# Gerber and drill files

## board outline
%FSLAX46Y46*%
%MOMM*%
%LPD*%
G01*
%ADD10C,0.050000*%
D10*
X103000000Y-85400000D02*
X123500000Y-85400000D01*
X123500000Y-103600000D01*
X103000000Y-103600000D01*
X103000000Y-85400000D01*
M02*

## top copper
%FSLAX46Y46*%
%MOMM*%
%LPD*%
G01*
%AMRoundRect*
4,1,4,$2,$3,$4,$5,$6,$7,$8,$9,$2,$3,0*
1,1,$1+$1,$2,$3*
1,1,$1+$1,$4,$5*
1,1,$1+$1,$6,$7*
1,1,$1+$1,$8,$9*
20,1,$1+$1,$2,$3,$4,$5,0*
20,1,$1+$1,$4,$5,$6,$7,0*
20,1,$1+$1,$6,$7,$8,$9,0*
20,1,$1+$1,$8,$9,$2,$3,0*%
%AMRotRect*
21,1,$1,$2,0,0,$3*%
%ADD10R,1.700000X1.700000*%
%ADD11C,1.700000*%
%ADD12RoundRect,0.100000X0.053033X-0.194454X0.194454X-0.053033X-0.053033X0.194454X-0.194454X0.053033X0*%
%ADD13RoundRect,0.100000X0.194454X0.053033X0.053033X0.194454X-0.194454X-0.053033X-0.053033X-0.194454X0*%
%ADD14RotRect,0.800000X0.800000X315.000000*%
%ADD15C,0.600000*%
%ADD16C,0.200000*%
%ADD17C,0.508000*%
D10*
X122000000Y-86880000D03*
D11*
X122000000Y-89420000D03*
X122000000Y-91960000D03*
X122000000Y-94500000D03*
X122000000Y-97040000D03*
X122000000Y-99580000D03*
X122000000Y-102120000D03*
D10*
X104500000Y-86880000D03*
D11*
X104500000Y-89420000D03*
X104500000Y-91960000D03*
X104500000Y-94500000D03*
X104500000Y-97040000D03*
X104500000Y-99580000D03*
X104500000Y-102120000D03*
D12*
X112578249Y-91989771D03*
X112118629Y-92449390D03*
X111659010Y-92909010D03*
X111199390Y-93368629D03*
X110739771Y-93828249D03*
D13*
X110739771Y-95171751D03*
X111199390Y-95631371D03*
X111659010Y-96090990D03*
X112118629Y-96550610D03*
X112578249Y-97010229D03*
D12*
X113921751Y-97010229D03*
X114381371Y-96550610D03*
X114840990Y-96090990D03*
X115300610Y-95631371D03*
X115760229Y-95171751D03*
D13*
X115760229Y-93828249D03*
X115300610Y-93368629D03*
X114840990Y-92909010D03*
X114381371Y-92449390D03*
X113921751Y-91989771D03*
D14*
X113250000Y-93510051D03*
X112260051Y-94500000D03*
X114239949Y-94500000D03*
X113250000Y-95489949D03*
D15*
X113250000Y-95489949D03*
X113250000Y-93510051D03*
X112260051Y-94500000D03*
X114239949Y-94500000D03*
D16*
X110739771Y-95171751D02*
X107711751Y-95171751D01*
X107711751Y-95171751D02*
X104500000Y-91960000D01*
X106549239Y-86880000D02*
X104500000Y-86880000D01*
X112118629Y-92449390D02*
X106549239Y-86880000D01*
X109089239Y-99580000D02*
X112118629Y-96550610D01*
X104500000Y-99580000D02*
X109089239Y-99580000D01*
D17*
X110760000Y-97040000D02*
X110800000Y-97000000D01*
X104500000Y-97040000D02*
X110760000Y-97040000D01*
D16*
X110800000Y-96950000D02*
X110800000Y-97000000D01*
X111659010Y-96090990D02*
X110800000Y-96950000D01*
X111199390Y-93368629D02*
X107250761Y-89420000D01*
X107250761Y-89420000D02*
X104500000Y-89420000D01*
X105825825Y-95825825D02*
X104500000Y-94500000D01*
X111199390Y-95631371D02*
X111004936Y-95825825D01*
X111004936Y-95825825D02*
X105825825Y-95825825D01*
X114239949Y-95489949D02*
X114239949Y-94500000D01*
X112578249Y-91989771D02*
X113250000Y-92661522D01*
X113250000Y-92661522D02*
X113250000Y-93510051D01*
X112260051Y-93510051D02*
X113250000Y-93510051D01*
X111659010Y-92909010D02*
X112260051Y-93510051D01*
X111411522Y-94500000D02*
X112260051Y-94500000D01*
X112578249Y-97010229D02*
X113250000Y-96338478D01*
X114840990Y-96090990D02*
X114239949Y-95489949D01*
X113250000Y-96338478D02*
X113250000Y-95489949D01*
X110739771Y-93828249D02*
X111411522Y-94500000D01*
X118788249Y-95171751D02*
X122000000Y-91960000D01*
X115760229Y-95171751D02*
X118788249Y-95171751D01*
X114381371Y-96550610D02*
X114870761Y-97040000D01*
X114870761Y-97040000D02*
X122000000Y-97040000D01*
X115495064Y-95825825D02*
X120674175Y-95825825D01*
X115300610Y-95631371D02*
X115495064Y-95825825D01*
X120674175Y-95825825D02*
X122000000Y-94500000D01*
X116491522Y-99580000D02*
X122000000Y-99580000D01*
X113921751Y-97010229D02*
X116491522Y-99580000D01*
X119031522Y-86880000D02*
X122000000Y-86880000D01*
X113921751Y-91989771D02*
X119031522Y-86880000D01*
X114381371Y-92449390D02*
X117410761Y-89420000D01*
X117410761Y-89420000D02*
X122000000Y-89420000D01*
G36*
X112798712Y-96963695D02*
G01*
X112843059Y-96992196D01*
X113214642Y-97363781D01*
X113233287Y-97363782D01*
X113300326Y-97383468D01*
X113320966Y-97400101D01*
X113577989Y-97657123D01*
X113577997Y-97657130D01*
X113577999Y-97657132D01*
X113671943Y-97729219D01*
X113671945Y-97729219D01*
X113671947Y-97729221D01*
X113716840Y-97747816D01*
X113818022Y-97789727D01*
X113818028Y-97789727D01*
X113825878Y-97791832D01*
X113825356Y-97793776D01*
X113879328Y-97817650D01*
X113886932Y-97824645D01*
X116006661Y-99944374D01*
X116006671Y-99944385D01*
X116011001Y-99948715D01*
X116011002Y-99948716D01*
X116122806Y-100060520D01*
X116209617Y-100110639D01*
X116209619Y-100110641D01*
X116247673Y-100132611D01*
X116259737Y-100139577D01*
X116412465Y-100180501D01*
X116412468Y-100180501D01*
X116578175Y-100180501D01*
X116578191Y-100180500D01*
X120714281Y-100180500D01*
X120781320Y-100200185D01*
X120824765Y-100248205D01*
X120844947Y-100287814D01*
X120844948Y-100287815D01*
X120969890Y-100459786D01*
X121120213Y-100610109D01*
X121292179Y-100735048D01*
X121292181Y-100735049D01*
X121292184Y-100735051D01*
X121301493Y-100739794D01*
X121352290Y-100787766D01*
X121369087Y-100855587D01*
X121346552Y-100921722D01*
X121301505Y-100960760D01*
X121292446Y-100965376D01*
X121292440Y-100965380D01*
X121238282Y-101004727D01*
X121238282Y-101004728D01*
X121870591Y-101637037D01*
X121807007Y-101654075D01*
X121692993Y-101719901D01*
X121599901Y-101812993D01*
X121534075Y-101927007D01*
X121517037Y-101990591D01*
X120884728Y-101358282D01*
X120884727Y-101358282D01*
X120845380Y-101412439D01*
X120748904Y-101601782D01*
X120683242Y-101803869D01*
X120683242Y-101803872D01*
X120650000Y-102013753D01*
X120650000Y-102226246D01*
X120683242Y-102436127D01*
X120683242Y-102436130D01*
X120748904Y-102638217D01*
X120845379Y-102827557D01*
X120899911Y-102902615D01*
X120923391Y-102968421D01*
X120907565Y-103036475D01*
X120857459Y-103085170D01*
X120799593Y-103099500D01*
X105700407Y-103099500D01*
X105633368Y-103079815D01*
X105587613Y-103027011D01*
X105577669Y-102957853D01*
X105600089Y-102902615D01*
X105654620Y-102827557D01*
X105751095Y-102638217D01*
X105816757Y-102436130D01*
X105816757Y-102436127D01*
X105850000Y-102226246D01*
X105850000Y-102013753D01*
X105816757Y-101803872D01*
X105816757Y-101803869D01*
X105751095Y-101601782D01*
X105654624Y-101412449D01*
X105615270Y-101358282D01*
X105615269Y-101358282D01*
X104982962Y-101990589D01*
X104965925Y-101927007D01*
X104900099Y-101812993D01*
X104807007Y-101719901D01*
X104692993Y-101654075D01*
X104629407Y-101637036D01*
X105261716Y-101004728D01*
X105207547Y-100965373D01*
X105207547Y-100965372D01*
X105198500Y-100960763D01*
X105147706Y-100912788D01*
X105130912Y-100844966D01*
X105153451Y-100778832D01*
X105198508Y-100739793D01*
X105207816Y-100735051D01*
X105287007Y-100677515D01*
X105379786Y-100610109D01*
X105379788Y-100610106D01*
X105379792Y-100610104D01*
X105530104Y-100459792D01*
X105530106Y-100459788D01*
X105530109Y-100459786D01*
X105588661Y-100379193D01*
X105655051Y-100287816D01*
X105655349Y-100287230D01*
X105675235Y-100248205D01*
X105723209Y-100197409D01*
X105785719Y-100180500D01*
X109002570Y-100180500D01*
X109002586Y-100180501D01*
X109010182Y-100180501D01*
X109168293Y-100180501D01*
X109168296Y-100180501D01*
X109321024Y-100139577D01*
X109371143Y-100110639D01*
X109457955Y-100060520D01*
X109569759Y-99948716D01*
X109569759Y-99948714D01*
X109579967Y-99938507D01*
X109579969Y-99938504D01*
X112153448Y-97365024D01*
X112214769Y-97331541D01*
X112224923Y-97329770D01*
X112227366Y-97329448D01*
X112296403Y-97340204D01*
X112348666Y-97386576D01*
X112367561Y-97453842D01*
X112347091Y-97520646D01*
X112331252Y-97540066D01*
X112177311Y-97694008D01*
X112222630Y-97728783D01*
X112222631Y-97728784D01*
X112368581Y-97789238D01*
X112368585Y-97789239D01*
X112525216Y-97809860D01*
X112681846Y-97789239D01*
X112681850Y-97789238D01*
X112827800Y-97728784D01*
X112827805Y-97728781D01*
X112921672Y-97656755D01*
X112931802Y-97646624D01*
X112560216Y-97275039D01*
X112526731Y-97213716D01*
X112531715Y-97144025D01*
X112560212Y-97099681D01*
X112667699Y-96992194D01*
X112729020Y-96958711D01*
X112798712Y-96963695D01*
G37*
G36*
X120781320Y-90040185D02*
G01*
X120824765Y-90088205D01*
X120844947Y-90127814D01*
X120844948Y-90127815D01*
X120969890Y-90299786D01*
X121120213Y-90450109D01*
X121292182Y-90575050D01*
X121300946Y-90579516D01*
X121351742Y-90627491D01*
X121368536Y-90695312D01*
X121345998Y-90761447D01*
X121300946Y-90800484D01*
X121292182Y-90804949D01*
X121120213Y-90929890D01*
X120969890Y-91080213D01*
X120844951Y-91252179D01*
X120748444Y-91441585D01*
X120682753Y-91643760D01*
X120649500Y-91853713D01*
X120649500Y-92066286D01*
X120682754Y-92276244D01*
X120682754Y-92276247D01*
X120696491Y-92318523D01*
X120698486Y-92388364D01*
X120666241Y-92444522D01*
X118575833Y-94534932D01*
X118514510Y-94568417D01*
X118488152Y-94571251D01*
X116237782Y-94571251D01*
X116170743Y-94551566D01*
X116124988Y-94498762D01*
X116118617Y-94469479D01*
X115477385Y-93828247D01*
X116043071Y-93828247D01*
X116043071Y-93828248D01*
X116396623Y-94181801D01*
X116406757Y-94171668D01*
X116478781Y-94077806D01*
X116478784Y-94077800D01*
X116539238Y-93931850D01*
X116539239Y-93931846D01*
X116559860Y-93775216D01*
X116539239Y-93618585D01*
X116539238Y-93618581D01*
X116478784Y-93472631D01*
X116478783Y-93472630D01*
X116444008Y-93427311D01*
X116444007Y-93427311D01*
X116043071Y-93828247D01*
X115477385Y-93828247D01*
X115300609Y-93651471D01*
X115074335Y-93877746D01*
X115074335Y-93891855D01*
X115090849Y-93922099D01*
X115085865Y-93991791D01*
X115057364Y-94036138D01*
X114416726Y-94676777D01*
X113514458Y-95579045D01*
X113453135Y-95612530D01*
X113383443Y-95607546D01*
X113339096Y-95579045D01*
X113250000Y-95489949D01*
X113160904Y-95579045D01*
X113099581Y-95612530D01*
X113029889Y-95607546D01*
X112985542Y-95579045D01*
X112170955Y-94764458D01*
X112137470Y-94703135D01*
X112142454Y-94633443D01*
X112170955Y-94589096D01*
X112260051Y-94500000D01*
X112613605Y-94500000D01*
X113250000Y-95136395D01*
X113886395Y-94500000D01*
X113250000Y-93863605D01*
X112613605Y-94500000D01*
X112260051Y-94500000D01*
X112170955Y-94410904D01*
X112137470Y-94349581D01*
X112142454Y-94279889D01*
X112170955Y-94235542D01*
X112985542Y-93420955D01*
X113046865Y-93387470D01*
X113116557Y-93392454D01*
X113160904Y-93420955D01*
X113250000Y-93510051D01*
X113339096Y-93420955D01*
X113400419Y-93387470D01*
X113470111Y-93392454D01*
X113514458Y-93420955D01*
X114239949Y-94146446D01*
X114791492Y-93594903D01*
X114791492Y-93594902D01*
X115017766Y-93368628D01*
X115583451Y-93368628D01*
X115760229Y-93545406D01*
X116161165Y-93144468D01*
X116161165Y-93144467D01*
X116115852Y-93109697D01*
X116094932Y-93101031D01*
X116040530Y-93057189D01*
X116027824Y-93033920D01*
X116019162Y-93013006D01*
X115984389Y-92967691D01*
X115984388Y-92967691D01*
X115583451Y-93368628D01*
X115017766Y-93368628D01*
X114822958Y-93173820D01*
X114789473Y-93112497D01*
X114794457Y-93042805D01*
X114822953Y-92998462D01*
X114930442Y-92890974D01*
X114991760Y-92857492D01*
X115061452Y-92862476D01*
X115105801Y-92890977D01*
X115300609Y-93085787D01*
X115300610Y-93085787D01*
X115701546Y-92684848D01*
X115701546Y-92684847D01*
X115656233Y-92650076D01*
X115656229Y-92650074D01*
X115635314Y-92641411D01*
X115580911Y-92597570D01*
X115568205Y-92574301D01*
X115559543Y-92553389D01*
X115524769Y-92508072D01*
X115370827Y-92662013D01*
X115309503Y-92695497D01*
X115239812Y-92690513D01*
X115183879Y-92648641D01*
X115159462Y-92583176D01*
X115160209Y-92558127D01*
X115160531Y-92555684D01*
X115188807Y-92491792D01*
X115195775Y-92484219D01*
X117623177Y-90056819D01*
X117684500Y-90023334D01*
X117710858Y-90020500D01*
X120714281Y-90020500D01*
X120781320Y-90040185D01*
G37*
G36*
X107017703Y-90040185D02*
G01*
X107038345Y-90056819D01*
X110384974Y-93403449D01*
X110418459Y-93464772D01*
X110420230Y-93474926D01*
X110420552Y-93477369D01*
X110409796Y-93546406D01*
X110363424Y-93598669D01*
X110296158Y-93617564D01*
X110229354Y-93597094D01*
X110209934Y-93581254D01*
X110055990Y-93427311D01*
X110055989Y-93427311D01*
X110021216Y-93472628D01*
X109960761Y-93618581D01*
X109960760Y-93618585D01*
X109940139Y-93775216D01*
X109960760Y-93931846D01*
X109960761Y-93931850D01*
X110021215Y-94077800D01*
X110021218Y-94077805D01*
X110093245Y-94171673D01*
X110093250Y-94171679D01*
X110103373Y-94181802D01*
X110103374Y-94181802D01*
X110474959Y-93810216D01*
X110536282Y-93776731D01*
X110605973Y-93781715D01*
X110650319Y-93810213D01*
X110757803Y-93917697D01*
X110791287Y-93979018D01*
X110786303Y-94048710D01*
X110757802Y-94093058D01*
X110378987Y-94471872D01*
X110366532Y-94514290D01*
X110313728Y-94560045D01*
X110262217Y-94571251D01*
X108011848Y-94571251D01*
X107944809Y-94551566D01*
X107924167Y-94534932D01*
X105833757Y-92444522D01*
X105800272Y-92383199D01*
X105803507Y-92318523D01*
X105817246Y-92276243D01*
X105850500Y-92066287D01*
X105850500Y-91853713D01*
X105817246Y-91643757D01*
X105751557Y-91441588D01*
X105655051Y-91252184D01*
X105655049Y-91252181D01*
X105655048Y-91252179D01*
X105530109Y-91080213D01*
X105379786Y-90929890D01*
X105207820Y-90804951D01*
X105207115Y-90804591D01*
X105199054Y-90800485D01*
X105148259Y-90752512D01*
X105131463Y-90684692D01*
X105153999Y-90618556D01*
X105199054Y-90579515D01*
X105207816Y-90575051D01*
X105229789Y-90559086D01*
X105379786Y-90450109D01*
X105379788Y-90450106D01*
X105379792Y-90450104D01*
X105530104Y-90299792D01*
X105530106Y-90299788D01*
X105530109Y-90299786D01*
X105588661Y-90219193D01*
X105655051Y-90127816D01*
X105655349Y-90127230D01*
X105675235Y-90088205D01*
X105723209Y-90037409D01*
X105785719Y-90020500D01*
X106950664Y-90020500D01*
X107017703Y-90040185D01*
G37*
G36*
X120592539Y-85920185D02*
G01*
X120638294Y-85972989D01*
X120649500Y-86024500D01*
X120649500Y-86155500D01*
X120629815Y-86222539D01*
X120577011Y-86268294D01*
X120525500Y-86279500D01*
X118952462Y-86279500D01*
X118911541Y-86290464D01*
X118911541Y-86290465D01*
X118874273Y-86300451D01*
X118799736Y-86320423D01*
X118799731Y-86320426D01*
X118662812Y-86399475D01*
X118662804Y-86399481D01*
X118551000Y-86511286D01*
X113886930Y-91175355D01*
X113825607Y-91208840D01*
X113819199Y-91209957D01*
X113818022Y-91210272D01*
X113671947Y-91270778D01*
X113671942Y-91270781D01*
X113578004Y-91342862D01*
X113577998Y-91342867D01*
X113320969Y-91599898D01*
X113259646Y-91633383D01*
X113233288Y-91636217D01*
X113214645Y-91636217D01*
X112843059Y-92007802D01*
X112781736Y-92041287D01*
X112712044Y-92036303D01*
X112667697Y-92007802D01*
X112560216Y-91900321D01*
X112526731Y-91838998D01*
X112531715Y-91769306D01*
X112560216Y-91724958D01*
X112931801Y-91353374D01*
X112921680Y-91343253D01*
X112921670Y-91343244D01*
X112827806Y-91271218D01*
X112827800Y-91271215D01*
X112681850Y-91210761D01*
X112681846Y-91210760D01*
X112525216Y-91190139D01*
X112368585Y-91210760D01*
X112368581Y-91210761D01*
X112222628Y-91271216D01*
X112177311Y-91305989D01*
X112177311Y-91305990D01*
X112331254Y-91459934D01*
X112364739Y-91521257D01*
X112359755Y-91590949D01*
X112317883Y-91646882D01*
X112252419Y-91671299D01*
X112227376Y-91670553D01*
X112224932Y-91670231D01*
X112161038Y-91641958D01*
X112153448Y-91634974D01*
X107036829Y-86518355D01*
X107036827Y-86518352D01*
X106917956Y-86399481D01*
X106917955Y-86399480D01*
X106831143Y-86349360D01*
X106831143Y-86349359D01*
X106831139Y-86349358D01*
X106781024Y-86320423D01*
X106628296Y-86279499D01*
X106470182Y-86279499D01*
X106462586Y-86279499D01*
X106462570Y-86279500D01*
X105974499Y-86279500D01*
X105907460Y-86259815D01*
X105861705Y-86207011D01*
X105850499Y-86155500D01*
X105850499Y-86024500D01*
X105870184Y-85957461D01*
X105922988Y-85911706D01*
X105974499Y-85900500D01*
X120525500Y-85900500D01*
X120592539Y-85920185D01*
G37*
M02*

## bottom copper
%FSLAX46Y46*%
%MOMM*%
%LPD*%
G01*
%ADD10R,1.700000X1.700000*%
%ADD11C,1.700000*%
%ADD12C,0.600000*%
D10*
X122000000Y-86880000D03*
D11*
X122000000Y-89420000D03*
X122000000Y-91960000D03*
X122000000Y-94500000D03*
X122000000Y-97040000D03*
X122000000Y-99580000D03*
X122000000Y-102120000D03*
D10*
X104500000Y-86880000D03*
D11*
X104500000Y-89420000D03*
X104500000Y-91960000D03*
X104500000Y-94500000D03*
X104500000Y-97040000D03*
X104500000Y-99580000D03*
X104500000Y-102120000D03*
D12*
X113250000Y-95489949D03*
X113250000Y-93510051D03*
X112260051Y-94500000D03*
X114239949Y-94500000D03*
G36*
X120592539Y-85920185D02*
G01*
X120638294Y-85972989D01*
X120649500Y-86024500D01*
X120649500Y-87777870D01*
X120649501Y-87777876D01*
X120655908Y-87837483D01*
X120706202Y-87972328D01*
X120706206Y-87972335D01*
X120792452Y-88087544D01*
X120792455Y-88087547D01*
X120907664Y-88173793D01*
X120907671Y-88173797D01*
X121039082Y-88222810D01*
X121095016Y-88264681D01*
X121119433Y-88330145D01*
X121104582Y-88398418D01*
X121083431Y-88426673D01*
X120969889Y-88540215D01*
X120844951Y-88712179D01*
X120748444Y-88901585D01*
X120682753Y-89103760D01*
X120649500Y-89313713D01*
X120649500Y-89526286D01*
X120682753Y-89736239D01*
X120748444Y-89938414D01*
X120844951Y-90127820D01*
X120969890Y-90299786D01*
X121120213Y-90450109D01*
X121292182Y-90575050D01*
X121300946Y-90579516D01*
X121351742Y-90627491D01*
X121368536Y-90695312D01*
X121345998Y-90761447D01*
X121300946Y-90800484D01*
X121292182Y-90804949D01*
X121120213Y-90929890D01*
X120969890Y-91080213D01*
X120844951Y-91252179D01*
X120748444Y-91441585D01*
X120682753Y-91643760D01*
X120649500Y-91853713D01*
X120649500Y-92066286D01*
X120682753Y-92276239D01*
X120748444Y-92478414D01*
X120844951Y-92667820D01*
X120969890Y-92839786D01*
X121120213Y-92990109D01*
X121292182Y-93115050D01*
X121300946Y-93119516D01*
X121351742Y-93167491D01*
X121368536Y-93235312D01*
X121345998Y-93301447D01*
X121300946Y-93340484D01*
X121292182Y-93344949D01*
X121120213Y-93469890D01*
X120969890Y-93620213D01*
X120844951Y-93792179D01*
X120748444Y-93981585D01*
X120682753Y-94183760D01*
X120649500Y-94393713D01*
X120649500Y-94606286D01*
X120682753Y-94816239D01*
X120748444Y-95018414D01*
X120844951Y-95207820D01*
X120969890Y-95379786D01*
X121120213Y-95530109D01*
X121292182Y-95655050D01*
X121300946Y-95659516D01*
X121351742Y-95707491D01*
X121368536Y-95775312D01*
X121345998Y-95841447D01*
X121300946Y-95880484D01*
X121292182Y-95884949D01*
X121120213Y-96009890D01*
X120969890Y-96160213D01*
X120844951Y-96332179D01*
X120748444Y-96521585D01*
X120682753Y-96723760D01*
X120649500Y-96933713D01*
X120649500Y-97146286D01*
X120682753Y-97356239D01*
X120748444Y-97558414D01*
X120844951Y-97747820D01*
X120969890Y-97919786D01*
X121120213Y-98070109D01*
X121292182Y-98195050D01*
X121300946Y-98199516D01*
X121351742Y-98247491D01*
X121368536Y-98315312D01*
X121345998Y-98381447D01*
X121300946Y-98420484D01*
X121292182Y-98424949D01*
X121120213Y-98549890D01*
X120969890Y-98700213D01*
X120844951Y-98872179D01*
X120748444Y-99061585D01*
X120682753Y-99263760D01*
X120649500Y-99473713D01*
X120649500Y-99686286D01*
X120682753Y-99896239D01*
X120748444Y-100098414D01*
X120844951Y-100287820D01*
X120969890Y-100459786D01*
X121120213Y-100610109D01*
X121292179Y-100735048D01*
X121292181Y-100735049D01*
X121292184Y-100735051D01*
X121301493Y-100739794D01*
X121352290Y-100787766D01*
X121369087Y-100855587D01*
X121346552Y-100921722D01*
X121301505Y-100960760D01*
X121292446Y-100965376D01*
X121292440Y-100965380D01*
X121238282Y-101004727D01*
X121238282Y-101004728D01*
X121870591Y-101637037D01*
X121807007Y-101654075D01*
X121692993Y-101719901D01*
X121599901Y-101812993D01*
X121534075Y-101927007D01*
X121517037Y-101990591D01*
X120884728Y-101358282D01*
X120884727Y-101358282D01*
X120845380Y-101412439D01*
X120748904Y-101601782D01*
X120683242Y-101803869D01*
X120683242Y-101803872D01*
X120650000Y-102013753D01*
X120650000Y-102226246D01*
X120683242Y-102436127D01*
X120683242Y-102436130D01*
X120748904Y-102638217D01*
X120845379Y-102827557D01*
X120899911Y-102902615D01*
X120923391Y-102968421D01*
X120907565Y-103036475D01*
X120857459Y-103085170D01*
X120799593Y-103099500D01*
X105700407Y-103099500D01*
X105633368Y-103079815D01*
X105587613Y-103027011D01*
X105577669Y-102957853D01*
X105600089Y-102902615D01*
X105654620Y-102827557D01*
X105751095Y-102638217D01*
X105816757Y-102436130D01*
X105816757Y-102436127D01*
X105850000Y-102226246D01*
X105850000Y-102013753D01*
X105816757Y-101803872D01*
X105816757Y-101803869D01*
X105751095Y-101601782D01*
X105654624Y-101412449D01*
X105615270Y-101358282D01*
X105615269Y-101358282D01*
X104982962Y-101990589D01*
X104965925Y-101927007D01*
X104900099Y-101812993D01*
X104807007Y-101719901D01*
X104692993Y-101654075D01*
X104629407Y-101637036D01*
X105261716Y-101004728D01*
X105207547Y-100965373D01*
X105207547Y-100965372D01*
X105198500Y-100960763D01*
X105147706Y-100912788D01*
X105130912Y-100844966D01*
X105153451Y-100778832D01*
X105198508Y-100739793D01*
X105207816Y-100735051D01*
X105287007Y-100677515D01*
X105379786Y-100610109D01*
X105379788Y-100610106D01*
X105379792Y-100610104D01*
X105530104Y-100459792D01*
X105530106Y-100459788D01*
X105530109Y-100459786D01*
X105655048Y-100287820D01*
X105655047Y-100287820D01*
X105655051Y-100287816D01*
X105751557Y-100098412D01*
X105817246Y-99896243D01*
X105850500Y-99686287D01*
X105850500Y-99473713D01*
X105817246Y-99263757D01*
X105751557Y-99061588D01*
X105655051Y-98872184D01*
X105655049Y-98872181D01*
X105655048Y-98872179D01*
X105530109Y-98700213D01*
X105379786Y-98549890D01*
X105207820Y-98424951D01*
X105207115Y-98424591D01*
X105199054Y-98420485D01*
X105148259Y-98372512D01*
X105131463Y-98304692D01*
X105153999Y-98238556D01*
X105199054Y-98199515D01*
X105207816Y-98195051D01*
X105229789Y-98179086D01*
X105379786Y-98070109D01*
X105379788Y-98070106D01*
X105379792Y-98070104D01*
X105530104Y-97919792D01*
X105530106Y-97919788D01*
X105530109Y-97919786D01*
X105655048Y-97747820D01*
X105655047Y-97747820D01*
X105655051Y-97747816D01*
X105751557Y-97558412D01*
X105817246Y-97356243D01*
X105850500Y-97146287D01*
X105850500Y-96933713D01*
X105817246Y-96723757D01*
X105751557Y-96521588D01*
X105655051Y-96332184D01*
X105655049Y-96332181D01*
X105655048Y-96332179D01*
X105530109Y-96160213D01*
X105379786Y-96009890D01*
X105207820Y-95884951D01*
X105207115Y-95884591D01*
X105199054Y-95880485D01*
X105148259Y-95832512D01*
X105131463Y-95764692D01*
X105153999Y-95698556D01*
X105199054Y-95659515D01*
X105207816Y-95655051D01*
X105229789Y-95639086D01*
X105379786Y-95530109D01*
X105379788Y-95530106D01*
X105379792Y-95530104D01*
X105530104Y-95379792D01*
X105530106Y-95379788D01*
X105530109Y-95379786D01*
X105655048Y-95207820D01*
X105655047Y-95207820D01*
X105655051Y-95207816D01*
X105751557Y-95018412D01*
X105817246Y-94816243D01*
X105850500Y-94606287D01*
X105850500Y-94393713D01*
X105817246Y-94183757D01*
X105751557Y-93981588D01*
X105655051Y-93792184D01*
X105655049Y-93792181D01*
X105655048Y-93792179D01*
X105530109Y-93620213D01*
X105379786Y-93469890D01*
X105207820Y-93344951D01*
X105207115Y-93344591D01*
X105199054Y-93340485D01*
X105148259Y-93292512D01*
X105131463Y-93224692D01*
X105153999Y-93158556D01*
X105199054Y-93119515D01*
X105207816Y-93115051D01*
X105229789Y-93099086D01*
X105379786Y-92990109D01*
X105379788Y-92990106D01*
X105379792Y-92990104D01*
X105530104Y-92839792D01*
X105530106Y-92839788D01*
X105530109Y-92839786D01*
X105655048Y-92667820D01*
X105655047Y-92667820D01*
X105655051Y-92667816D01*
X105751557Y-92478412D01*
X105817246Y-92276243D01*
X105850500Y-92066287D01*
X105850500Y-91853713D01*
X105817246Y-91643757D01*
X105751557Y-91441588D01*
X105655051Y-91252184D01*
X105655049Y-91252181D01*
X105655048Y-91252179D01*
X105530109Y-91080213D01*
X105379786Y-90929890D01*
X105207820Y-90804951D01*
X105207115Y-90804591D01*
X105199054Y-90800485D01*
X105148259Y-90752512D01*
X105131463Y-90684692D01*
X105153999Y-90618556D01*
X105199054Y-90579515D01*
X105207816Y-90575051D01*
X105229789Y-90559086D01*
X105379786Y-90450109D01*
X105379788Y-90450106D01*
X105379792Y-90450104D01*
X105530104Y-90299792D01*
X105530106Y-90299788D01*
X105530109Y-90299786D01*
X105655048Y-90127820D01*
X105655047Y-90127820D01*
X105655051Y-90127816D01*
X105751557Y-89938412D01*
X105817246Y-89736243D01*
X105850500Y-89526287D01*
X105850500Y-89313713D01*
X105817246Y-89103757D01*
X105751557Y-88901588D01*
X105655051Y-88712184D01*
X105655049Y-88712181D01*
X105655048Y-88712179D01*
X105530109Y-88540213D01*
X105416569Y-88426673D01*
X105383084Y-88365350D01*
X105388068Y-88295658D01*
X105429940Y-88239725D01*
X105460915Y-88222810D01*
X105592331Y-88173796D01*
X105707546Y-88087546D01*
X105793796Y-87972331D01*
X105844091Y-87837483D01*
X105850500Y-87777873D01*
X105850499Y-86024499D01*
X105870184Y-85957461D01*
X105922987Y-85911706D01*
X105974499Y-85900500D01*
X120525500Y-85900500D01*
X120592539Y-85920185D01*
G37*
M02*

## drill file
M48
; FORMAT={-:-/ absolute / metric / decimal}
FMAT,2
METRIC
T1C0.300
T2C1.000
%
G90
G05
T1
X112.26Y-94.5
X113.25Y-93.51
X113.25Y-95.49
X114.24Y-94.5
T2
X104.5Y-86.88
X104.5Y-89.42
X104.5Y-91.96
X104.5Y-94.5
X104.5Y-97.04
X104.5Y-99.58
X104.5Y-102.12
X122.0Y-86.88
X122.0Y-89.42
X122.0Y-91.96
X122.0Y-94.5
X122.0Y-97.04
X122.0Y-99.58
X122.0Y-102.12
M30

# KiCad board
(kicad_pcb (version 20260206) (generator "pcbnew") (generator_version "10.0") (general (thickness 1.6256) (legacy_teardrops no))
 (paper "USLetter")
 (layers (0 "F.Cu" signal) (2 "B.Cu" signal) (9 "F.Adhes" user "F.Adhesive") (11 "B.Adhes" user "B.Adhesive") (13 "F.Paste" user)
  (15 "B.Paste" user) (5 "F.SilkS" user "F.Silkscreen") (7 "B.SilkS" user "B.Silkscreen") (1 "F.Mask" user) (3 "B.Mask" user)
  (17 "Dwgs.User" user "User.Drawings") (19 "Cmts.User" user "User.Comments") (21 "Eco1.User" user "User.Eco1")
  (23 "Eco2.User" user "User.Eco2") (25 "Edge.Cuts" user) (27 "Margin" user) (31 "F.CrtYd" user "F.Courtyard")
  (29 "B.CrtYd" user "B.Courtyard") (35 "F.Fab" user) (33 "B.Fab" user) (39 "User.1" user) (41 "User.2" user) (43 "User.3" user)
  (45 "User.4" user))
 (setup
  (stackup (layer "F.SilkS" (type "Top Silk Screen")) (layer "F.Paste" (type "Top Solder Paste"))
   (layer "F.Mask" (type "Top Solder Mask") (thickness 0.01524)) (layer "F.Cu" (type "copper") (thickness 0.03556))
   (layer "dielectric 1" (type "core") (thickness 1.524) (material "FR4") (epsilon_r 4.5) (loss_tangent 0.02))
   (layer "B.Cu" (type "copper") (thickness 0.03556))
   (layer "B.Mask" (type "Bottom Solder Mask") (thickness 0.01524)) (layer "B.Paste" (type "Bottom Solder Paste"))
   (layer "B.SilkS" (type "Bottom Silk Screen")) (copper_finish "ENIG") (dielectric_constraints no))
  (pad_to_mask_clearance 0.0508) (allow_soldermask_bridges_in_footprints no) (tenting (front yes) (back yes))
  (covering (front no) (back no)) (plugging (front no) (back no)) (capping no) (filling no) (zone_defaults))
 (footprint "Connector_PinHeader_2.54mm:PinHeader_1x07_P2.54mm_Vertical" (layer "F.Cu") (at 122 86.88)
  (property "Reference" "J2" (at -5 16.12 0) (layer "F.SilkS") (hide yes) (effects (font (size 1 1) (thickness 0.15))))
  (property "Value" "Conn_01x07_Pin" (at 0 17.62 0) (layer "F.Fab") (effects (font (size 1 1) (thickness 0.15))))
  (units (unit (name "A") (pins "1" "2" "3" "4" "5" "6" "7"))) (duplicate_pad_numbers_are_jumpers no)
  (pad "1" thru_hole rect (at 0 0) (size 1.7 1.7) (drill 1) (layers "*.Cu" "*.Mask") (remove_unused_layers no) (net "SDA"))
  (pad "2" thru_hole circle (at 0 2.54) (size 1.7 1.7) (drill 1) (layers "*.Cu" "*.Mask") (remove_unused_layers no) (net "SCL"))
  (pad "3" thru_hole circle (at 0 5.08) (size 1.7 1.7) (drill 1) (layers "*.Cu" "*.Mask") (remove_unused_layers no) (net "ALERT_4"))
  (pad "4" thru_hole circle (at 0 7.62) (size 1.7 1.7) (drill 1) (layers "*.Cu" "*.Mask") (remove_unused_layers no) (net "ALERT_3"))
  (pad "5" thru_hole circle (at 0 10.16) (size 1.7 1.7) (drill 1) (layers "*.Cu" "*.Mask") (remove_unused_layers no) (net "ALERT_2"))
  (pad "6" thru_hole circle (at 0 12.7) (size 1.7 1.7) (drill 1) (layers "*.Cu" "*.Mask") (remove_unused_layers no) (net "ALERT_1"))
  (pad "7" thru_hole circle (at 0 15.24) (size 1.7 1.7) (drill 1) (layers "*.Cu" "*.Mask") (remove_unused_layers no) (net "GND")))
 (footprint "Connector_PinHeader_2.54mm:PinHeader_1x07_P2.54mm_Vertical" (layer "F.Cu") (at 104.5 86.88)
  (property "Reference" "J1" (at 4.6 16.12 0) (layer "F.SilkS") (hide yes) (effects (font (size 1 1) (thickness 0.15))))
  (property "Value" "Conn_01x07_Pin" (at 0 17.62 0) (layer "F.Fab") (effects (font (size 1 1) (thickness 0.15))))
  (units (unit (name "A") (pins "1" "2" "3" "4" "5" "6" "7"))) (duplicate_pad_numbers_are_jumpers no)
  (pad "1" thru_hole rect (at 0 0) (size 1.7 1.7) (drill 1) (layers "*.Cu" "*.Mask") (remove_unused_layers no) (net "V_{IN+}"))
  (pad "2" thru_hole circle (at 0 2.54) (size 1.7 1.7) (drill 1) (layers "*.Cu" "*.Mask") (remove_unused_layers no) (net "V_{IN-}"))
  (pad "3" thru_hole circle (at 0 5.08) (size 1.7 1.7) (drill 1) (layers "*.Cu" "*.Mask") (remove_unused_layers no) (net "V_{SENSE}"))
  (pad "4" thru_hole circle (at 0 7.62) (size 1.7 1.7) (drill 1) (layers "*.Cu" "*.Mask") (remove_unused_layers no) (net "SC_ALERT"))
  (pad "5" thru_hole circle (at 0 10.16) (size 1.7 1.7) (drill 1) (layers "*.Cu" "*.Mask") (remove_unused_layers no) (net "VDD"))
  (pad "6" thru_hole circle (at 0 12.7) (size 1.7 1.7) (drill 1) (layers "*.Cu" "*.Mask") (remove_unused_layers no) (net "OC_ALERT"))
  (pad "7" thru_hole circle (at 0 15.24) (size 1.7 1.7) (drill 1) (layers "*.Cu" "*.Mask") (remove_unused_layers no) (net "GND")))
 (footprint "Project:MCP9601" (layer "F.Cu") (at 113.25 94.5 -45)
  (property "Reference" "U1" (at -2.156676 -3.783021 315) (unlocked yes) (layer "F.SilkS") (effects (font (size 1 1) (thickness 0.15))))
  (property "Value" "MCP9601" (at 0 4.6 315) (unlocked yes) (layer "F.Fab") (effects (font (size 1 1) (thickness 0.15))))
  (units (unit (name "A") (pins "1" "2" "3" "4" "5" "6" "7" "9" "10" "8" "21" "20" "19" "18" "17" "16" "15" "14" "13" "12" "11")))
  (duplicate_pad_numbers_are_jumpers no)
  (pad "1" smd roundrect (at -2.25 -1.3 45) (size 0.4 0.55) (layers "F.Cu" "F.Mask" "F.Paste") (roundrect_rratio 0.25) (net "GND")
   (solder_paste_margin_ratio -0.15))
  (pad "2" smd roundrect (at -2.25 -0.65 45) (size 0.4 0.55) (layers "F.Cu" "F.Mask" "F.Paste") (roundrect_rratio 0.25) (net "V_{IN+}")
   (solder_paste_margin_ratio -0.15))
  (pad "3" smd roundrect (at -2.25 0 45) (size 0.4 0.55) (layers "F.Cu" "F.Mask" "F.Paste") (roundrect_rratio 0.25) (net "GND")
   (solder_paste_margin_ratio -0.15))
  (pad "4" smd roundrect (at -2.25 0.65 45) (size 0.4 0.55) (layers "F.Cu" "F.Mask" "F.Paste") (roundrect_rratio 0.25) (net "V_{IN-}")
   (solder_paste_margin_ratio -0.15))
  (pad "5" smd roundrect (at -2.25 1.3 45) (size 0.4 0.55) (layers "F.Cu" "F.Mask" "F.Paste") (roundrect_rratio 0.25) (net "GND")
   (solder_paste_margin_ratio -0.15))
  (pad "6" smd roundrect (at -1.3 2.25 135) (size 0.4 0.55) (layers "F.Cu" "F.Mask" "F.Paste") (roundrect_rratio 0.25) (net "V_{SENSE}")
   (solder_paste_margin_ratio -0.15))
  (pad "7" smd roundrect (at -0.65 2.25 135) (size 0.4 0.55) (layers "F.Cu" "F.Mask" "F.Paste") (roundrect_rratio 0.25) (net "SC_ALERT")
   (solder_paste_margin_ratio -0.15))
  (pad "8" smd roundrect (at 0 2.25 135) (size 0.4 0.55) (layers "F.Cu" "F.Mask" "F.Paste") (roundrect_rratio 0.25) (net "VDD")
   (solder_paste_margin_ratio -0.15))
  (pad "9" smd roundrect (at 0.65 2.25 135) (size 0.4 0.55) (layers "F.Cu" "F.Mask" "F.Paste") (roundrect_rratio 0.25) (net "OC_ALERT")
   (solder_paste_margin_ratio -0.15))
  (pad "10" smd roundrect (at 1.3 2.25 135) (size 0.4 0.55) (layers "F.Cu" "F.Mask" "F.Paste") (roundrect_rratio 0.25) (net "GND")
   (solder_paste_margin_ratio -0.15))
  (pad "11" smd roundrect (at 2.25 1.3 45) (size 0.4 0.55) (layers "F.Cu" "F.Mask" "F.Paste") (roundrect_rratio 0.25) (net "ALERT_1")
   (solder_paste_margin_ratio -0.15))
  (pad "12" smd roundrect (at 2.25 0.65 45) (size 0.4 0.55) (layers "F.Cu" "F.Mask" "F.Paste") (roundrect_rratio 0.25) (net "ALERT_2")
   (solder_paste_margin_ratio -0.15))
  (pad "13" smd roundrect (at 2.25 0 45) (size 0.4 0.55) (layers "F.Cu" "F.Mask" "F.Paste") (roundrect_rratio 0.25) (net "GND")
   (solder_paste_margin_ratio -0.15))
  (pad "14" smd roundrect (at 2.25 -0.65 45) (size 0.4 0.55) (layers "F.Cu" "F.Mask" "F.Paste") (roundrect_rratio 0.25) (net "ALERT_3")
   (solder_paste_margin_ratio -0.15))
  (pad "15" smd roundrect (at 2.25 -1.3 45) (size 0.4 0.55) (layers "F.Cu" "F.Mask" "F.Paste") (roundrect_rratio 0.25) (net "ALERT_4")
   (solder_paste_margin_ratio -0.15))
  (pad "16" smd roundrect (at 1.3 -2.25 135) (size 0.4 0.55) (layers "F.Cu" "F.Mask" "F.Paste") (roundrect_rratio 0.25) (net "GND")
   (solder_paste_margin_ratio -0.15))
  (pad "17" smd roundrect (at 0.65 -2.25 135) (size 0.4 0.55) (layers "F.Cu" "F.Mask" "F.Paste") (roundrect_rratio 0.25) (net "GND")
   (solder_paste_margin_ratio -0.15))
  (pad "18" smd roundrect (at 0 -2.25 135) (size 0.4 0.55) (layers "F.Cu" "F.Mask" "F.Paste") (roundrect_rratio 0.25) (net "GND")
   (solder_paste_margin_ratio -0.15))
  (pad "19" smd roundrect (at -0.65 -2.25 135) (size 0.4 0.55) (layers "F.Cu" "F.Mask" "F.Paste") (roundrect_rratio 0.25) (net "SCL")
   (solder_paste_margin_ratio -0.15))
  (pad "20" smd roundrect (at -1.3 -2.25 135) (size 0.4 0.55) (layers "F.Cu" "F.Mask" "F.Paste") (roundrect_rratio 0.25) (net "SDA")
   (solder_paste_margin_ratio -0.15))
  (pad "21" smd rect (at -0.7 -0.7 315) (size 0.8 0.8) (layers "F.Cu" "F.Mask" "F.Paste") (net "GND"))
  (pad "21" smd rect (at -0.7 0.7 315) (size 0.8 0.8) (layers "F.Cu" "F.Mask" "F.Paste") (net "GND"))
  (pad "21" smd rect (at 0.7 -0.7 315) (size 0.8 0.8) (layers "F.Cu" "F.Mask" "F.Paste") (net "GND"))
  (pad "21" smd rect (at 0.7 0.7 315) (size 0.8 0.8) (layers "F.Cu" "F.Mask" "F.Paste") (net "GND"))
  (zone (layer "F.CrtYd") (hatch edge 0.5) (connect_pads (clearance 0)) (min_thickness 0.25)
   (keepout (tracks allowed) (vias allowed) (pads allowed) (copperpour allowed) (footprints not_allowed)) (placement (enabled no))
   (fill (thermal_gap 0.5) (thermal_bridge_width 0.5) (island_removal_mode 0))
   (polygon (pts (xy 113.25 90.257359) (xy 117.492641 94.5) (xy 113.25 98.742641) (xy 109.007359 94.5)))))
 (gr_rect (start 103 85.4) (end 123.5 103.6) (stroke (width 0.05) (type default)) (fill no) (layer "Edge.Cuts"))
 (segment (start 110.739771 95.171751) (end 107.711751 95.171751) (width 0.2) (layer "F.Cu") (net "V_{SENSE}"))
 (segment (start 107.711751 95.171751) (end 104.5 91.96) (width 0.2) (layer "F.Cu") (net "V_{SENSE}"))
 (segment (start 106.549239 86.88) (end 104.5 86.88) (width 0.2) (layer "F.Cu") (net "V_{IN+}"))
 (segment (start 112.118629 92.44939) (end 106.549239 86.88) (width 0.2) (layer "F.Cu") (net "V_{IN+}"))
 (segment (start 109.089239 99.58) (end 112.118629 96.55061) (width 0.2) (layer "F.Cu") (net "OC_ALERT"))
 (segment (start 104.5 99.58) (end 109.089239 99.58) (width 0.2) (layer "F.Cu") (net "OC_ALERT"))
 (segment (start 110.76 97.04) (end 110.8 97) (width 0.508) (layer "F.Cu") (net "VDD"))
 (segment (start 104.5 97.04) (end 110.76 97.04) (width 0.508) (layer "F.Cu") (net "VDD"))
 (segment (start 110.8 96.95) (end 110.8 97) (width 0.2) (layer "F.Cu") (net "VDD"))
 (segment (start 111.65901 96.09099) (end 110.8 96.95) (width 0.2) (layer "F.Cu") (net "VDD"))
 (segment (start 111.19939 93.368629) (end 107.250761 89.42) (width 0.2) (layer "F.Cu") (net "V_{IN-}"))
 (segment (start 107.250761 89.42) (end 104.5 89.42) (width 0.2) (layer "F.Cu") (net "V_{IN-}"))
 (segment (start 105.825825 95.825825) (end 104.5 94.5) (width 0.2) (layer "F.Cu") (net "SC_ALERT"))
 (segment (start 111.19939 95.631371) (end 111.004936 95.825825) (width 0.2) (layer "F.Cu") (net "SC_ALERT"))
 (segment (start 111.004936 95.825825) (end 105.825825 95.825825) (width 0.2) (layer "F.Cu") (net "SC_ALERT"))
 (segment (start 114.239949 95.489949) (end 114.239949 94.5) (width 0.2) (layer "F.Cu") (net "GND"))
 (segment (start 112.578249 91.989771) (end 113.25 92.661522) (width 0.2) (layer "F.Cu") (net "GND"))
 (segment (start 113.25 92.661522) (end 113.25 93.510051) (width 0.2) (layer "F.Cu") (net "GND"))
 (segment (start 112.260051 93.510051) (end 113.25 93.510051) (width 0.2) (layer "F.Cu") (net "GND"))
 (segment (start 111.65901 92.90901) (end 112.260051 93.510051) (width 0.2) (layer "F.Cu") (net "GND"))
 (segment (start 111.411522 94.5) (end 112.260051 94.5) (width 0.2) (layer "F.Cu") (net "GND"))
 (segment (start 112.578249 97.010229) (end 113.25 96.338478) (width 0.2) (layer "F.Cu") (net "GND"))
 (segment (start 114.84099 96.09099) (end 114.239949 95.489949) (width 0.2) (layer "F.Cu") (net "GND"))
 (segment (start 113.25 96.338478) (end 113.25 95.489949) (width 0.2) (layer "F.Cu") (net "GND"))
 (segment (start 110.739771 93.828249) (end 111.411522 94.5) (width 0.2) (layer "F.Cu") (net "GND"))
 (via (at 113.25 95.489949) (size 0.6) (drill 0.3) (layers "F.Cu" "B.Cu") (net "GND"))
 (via (at 113.25 93.510051) (size 0.6) (drill 0.3) (layers "F.Cu" "B.Cu") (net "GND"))
 (via (at 112.260051 94.5) (size 0.6) (drill 0.3) (layers "F.Cu" "B.Cu") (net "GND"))
 (via (at 114.239949 94.5) (size 0.6) (drill 0.3) (layers "F.Cu" "B.Cu") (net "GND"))
 (segment (start 118.788249 95.171751) (end 122 91.96) (width 0.2) (layer "F.Cu") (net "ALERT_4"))
 (segment (start 115.760229 95.171751) (end 118.788249 95.171751) (width 0.2) (layer "F.Cu") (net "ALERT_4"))
 (segment (start 114.381371 96.55061) (end 114.870761 97.04) (width 0.2) (layer "F.Cu") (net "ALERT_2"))
 (segment (start 114.870761 97.04) (end 122 97.04) (width 0.2) (layer "F.Cu") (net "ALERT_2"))
 (segment (start 115.495064 95.825825) (end 120.674175 95.825825) (width 0.2) (layer "F.Cu") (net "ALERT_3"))
 (segment (start 115.30061 95.631371) (end 115.495064 95.825825) (width 0.2) (layer "F.Cu") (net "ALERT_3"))
 (segment (start 120.674175 95.825825) (end 122 94.5) (width 0.2) (layer "F.Cu") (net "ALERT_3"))
 (segment (start 116.491522 99.58) (end 122 99.58) (width 0.2) (layer "F.Cu") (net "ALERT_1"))
 (segment (start 113.921751 97.010229) (end 116.491522 99.58) (width 0.2) (layer "F.Cu") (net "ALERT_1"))
 (segment (start 119.031522 86.88) (end 122 86.88) (width 0.2) (layer "F.Cu") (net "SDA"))
 (segment (start 113.921751 91.989771) (end 119.031522 86.88) (width 0.2) (layer "F.Cu") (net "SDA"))
 (segment (start 114.381371 92.44939) (end 117.410761 89.42) (width 0.2) (layer "F.Cu") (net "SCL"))
 (segment (start 117.410761 89.42) (end 122 89.42) (width 0.2) (layer "F.Cu") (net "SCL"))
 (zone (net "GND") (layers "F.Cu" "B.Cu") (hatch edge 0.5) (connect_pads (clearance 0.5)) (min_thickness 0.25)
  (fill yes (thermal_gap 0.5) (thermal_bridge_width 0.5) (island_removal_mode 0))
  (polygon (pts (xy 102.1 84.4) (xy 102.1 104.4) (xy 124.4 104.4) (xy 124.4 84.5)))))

